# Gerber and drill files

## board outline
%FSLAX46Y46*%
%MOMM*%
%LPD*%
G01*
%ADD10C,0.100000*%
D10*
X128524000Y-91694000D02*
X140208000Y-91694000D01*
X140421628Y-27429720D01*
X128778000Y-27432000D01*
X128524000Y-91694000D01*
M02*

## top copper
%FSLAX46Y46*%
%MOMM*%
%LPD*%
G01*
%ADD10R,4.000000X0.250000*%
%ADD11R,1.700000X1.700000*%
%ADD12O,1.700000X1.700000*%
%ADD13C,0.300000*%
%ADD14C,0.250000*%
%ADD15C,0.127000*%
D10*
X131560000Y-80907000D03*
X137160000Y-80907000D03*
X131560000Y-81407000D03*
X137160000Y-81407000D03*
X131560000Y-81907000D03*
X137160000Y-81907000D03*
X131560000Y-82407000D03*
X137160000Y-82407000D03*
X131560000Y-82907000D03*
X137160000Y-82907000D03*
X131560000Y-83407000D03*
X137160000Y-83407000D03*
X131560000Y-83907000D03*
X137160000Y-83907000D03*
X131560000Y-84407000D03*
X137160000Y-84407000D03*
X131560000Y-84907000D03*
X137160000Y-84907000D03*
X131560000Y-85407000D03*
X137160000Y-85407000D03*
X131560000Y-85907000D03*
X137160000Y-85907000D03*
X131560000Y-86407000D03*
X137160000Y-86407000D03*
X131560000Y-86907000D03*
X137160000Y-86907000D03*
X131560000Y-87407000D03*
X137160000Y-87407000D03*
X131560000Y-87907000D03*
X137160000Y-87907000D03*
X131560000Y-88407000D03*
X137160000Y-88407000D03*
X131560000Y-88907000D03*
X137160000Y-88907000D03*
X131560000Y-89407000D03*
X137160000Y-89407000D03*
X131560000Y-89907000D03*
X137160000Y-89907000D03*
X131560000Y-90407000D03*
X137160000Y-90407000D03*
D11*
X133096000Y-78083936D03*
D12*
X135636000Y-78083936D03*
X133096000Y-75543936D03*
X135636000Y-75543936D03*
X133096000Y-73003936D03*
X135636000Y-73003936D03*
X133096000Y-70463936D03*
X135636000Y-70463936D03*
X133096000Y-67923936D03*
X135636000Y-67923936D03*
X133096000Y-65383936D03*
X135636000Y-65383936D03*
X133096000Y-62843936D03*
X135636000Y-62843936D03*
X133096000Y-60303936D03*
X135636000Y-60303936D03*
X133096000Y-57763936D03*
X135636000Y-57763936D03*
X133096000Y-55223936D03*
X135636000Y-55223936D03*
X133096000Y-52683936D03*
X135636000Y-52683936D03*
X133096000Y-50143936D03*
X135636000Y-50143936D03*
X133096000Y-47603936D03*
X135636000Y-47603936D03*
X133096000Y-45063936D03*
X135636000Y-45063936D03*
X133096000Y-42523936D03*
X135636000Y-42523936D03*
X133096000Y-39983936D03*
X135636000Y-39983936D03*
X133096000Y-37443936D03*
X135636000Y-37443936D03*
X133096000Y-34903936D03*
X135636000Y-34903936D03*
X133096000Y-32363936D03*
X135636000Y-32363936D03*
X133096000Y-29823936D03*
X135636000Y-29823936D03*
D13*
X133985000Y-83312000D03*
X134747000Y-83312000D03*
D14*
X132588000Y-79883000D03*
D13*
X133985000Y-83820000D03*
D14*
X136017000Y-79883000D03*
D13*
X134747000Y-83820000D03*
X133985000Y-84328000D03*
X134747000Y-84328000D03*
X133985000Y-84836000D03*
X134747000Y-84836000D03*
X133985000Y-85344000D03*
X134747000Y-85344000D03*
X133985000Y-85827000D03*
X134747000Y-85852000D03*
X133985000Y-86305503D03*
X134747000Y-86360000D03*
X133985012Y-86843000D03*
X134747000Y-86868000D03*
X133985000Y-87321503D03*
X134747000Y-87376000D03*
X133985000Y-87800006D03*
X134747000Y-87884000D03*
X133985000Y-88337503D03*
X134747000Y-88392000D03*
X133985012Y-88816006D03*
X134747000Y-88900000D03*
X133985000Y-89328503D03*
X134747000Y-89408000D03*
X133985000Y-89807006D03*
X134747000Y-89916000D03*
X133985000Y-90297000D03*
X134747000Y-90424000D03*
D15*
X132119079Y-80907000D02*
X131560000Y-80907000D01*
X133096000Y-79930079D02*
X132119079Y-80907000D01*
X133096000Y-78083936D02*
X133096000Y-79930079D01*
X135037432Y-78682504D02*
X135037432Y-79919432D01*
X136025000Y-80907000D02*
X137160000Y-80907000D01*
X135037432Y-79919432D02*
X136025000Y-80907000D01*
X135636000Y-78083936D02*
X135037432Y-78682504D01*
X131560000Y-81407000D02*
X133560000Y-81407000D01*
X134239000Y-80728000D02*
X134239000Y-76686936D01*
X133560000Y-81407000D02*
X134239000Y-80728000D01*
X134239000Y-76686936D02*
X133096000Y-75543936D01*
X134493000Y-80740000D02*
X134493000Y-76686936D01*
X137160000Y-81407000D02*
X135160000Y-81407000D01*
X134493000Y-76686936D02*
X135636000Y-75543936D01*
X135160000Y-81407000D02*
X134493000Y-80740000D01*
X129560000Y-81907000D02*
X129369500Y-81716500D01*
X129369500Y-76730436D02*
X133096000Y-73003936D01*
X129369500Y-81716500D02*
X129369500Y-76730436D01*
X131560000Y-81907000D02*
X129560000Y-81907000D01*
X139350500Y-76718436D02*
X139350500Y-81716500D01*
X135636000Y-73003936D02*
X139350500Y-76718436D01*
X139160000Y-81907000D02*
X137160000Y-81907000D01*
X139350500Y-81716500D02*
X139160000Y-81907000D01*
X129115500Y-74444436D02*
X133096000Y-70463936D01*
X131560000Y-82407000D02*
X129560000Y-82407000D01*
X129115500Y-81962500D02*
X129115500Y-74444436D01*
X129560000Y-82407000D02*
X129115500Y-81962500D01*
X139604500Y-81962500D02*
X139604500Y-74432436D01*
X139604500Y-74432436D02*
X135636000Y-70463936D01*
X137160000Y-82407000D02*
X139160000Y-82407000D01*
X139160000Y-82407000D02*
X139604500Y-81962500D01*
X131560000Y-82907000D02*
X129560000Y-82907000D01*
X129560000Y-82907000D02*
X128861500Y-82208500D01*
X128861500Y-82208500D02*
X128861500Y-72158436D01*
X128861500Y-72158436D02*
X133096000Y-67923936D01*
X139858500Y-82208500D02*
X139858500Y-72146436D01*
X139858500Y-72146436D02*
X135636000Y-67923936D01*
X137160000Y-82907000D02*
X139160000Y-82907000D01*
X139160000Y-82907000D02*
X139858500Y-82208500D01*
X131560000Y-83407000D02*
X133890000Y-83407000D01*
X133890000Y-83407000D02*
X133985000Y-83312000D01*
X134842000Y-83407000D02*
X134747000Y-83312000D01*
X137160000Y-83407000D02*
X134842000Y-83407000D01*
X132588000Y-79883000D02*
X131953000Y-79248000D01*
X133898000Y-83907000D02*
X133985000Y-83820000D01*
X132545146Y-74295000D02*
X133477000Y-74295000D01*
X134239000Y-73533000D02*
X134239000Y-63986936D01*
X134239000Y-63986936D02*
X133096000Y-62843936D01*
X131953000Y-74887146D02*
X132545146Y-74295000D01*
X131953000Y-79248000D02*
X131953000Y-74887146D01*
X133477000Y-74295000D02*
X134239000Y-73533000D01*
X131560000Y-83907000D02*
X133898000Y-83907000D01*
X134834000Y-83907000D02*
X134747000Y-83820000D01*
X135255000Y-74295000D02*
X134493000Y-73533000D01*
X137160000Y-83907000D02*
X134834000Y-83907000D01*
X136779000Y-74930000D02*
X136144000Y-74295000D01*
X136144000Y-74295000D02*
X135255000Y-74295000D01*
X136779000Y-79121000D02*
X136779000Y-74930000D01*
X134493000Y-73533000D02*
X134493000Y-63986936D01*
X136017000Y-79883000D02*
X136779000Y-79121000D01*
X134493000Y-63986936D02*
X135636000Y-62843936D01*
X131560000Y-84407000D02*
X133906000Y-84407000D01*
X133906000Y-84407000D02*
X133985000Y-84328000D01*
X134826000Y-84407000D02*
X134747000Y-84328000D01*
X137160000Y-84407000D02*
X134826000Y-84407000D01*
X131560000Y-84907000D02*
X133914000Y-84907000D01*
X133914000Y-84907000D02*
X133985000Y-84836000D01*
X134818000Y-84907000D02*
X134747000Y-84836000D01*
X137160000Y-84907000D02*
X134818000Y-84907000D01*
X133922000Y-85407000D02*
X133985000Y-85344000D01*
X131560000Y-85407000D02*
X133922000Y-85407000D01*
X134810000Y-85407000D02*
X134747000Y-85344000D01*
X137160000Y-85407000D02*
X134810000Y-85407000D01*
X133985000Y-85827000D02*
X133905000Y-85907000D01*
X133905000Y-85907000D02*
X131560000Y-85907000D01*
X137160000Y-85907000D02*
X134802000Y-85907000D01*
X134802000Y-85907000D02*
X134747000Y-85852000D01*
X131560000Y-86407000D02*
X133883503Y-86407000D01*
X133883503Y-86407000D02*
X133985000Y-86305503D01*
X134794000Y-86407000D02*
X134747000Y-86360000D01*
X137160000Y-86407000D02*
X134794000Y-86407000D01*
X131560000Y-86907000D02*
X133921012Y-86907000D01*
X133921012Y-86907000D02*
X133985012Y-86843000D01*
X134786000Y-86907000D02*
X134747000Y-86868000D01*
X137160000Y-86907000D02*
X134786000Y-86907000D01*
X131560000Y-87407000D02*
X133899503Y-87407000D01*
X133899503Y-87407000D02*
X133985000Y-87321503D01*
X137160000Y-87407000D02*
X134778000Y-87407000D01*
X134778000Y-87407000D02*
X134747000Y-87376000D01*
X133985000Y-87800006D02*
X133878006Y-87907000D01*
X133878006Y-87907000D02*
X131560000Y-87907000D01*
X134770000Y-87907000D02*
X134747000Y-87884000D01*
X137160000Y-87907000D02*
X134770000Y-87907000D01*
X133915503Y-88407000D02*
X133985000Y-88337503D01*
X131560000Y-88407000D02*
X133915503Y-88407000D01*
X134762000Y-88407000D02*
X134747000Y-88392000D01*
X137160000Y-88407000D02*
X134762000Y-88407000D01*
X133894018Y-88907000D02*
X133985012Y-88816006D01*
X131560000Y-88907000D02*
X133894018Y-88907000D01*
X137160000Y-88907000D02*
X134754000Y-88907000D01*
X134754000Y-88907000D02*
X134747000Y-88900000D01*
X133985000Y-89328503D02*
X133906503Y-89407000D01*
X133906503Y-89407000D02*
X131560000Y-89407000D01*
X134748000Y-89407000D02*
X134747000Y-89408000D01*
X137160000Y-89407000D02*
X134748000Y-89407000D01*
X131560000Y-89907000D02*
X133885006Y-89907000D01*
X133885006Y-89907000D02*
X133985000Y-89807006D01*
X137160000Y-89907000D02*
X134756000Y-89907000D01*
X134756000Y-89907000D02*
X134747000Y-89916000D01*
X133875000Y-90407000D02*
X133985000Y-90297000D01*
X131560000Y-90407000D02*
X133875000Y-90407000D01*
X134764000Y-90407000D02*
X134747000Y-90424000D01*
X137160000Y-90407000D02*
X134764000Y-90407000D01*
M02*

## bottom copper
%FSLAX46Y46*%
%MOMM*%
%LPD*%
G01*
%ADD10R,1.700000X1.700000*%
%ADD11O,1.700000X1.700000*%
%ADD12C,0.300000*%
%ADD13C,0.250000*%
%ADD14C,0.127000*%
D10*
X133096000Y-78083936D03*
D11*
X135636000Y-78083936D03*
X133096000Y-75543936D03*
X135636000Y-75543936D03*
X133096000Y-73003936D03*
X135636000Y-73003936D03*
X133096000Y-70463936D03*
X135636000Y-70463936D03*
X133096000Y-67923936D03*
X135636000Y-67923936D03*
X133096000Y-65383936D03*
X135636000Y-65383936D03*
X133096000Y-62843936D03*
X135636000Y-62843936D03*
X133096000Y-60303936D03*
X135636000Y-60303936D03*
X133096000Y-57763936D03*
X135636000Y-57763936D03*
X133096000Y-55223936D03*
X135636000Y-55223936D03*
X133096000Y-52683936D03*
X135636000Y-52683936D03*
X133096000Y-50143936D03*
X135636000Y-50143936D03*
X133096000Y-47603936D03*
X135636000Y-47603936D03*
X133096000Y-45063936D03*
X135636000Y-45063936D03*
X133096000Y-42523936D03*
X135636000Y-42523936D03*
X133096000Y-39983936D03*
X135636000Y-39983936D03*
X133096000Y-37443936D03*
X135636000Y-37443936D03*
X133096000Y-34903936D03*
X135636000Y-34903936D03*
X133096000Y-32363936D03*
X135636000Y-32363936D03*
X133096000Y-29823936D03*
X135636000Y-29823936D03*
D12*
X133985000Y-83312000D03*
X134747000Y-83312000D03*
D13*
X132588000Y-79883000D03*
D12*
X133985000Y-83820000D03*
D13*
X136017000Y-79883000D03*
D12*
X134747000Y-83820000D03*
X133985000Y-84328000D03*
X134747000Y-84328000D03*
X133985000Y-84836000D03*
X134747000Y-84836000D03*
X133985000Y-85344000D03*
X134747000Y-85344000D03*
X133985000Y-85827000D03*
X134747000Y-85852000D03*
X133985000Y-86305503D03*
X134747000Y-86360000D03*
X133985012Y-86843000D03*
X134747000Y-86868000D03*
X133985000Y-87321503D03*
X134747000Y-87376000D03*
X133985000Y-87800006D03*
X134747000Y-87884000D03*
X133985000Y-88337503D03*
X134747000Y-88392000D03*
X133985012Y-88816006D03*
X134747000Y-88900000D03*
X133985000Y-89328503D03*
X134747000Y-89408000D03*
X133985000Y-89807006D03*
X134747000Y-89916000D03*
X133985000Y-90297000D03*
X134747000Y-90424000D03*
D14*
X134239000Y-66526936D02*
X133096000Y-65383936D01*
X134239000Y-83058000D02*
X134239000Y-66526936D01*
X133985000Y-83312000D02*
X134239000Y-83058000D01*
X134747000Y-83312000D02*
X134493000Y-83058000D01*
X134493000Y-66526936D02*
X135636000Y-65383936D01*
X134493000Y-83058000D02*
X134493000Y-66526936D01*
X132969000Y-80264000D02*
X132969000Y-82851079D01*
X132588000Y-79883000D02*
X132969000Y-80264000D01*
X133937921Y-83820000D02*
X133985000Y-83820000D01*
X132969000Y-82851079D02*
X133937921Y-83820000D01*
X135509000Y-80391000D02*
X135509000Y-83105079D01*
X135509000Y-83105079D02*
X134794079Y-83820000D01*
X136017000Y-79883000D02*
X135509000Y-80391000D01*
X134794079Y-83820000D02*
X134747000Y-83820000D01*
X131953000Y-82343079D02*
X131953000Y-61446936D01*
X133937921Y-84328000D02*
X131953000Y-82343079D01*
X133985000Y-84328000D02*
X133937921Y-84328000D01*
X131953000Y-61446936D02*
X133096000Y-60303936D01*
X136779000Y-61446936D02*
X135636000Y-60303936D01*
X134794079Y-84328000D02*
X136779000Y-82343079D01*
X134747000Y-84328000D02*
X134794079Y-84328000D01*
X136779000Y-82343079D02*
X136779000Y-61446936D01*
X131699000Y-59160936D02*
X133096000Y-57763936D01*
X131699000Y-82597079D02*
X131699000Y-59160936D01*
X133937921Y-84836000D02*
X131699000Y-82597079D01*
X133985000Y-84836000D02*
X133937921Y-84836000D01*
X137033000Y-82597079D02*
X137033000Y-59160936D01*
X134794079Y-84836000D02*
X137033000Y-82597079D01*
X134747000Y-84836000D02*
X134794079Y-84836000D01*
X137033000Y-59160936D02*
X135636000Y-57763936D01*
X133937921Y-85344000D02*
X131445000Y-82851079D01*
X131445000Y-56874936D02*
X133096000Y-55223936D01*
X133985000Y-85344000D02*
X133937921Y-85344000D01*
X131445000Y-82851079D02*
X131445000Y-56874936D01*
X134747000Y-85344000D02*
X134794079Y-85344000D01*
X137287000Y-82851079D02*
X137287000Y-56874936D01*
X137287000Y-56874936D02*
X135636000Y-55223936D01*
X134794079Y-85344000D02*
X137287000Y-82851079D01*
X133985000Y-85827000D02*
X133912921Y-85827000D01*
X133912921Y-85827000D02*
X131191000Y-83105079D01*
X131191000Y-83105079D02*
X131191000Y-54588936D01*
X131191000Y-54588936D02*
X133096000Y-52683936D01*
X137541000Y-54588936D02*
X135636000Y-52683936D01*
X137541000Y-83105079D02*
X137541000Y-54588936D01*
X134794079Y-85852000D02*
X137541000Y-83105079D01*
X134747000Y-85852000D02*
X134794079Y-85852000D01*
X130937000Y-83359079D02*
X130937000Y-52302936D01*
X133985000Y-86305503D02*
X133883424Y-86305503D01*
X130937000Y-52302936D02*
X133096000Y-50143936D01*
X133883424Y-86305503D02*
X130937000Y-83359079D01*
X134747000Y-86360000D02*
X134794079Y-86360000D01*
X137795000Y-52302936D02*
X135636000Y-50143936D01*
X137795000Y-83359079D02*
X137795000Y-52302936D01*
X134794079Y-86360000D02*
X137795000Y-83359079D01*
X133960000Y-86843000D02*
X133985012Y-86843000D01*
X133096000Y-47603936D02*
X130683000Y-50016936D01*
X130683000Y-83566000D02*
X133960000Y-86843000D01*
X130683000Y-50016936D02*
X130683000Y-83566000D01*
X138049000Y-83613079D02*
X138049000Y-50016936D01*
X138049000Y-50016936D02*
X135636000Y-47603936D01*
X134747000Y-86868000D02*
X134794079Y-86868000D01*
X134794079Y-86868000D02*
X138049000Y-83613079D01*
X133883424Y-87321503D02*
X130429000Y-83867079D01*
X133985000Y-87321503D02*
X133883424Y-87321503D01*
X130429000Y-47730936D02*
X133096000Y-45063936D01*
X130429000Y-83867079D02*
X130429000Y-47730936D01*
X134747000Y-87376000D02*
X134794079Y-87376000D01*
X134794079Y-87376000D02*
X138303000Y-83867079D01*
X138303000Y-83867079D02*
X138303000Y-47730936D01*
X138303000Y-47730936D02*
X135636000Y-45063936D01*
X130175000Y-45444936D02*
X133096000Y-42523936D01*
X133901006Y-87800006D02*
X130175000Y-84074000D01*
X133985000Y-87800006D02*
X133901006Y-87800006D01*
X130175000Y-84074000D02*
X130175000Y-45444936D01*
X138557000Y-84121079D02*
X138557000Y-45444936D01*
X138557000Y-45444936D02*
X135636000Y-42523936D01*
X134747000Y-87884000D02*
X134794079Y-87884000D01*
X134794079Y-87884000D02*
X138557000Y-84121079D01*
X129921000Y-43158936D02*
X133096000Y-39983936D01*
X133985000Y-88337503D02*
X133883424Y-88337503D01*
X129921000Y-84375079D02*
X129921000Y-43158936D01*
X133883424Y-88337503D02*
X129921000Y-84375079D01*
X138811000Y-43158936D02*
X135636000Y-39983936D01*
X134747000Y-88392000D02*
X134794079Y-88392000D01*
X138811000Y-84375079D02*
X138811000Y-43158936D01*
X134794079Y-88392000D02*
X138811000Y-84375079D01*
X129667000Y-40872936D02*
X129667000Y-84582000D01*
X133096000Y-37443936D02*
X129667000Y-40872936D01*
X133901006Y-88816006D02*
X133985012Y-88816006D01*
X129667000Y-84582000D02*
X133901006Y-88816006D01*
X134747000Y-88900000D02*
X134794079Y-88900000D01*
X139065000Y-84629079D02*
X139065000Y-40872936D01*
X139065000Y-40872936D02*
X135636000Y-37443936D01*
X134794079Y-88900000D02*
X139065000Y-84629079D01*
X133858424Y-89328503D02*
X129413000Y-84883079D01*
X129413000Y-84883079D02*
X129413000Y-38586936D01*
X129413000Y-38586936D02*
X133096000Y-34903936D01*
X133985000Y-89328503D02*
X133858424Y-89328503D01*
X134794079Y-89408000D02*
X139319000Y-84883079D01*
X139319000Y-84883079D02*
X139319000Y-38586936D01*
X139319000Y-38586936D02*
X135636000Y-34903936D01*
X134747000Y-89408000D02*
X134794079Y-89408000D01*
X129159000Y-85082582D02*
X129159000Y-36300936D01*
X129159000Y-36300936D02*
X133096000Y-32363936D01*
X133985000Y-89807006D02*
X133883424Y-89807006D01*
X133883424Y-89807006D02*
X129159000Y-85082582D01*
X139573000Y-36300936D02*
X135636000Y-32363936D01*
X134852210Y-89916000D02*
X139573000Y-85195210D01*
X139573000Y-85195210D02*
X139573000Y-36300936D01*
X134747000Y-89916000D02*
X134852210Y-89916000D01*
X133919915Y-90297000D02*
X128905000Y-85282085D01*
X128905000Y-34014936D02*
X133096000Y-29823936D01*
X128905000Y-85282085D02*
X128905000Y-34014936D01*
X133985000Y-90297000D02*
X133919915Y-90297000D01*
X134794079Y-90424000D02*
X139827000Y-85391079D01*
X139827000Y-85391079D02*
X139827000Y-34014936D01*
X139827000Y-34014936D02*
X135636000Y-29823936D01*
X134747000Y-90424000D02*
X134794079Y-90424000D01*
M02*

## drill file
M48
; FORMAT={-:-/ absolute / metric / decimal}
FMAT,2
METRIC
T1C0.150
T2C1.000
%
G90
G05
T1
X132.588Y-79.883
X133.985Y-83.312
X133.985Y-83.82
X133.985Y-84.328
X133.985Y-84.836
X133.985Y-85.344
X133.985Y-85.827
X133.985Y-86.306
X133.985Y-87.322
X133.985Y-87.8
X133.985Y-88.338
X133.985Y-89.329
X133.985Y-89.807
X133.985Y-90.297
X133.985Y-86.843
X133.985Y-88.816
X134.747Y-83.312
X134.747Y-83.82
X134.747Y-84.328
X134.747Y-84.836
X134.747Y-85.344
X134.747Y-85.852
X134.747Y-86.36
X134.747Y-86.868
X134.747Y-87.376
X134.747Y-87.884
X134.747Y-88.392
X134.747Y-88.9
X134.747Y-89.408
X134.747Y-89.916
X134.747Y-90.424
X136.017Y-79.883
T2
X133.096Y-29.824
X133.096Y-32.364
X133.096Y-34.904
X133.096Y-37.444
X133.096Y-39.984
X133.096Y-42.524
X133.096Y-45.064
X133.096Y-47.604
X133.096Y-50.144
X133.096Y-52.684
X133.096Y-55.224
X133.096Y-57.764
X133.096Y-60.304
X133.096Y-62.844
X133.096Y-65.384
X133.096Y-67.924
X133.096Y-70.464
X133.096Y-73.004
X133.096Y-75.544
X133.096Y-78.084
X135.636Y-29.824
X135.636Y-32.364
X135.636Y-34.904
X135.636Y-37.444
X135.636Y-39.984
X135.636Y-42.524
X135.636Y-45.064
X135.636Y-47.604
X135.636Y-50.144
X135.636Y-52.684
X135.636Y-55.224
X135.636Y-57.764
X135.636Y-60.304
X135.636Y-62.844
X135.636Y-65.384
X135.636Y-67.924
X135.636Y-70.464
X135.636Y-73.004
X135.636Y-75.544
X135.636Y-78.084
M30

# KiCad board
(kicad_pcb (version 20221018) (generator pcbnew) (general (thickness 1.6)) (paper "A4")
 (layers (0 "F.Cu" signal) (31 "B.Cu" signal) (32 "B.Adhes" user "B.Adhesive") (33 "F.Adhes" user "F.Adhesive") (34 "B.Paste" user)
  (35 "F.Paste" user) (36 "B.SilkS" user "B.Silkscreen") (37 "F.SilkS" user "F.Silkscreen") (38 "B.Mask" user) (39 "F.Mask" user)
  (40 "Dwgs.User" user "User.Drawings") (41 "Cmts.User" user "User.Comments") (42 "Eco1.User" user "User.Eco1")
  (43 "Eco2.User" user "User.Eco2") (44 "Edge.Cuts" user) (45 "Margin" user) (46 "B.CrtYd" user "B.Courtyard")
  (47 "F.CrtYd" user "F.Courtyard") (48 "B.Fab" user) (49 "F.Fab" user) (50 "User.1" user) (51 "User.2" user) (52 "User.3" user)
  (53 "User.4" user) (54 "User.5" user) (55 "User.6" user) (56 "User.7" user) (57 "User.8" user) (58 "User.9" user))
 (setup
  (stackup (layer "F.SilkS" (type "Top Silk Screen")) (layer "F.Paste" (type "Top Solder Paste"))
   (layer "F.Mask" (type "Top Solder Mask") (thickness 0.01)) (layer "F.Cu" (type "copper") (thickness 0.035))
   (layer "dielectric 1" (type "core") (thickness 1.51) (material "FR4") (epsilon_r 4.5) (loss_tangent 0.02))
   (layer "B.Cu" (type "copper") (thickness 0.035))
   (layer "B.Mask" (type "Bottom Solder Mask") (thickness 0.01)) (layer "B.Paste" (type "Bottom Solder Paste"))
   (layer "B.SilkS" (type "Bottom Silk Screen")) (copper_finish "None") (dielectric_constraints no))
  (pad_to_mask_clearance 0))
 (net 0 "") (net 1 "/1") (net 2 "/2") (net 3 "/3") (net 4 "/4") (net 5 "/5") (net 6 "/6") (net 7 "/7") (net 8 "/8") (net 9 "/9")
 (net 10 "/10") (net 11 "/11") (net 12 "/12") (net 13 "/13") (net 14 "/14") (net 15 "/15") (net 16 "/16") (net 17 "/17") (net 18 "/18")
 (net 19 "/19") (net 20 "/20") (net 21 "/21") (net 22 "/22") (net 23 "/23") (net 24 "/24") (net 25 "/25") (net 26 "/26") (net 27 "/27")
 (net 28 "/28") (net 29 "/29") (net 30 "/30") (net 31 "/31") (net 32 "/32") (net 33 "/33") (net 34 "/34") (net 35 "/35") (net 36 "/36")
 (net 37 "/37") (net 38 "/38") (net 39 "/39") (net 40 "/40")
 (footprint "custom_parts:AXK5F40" (layer "F.Cu") (at 134.36 85.657)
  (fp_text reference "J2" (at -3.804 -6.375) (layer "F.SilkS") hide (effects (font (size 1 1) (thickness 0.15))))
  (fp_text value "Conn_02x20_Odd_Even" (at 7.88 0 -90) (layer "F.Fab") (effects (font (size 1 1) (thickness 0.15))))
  (pad "1" smd rect (at -2.8 -4.75 270) (size 0.25 4) (layers "F.Cu" "F.Paste" "F.Mask") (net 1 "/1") (thermal_bridge_angle 45))
  (pad "2" smd rect (at 2.8 -4.75 270) (size 0.25 4) (layers "F.Cu" "F.Paste" "F.Mask") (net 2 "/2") (thermal_bridge_angle 45))
  (pad "3" smd rect (at -2.8 -4.25 270) (size 0.25 4) (layers "F.Cu" "F.Paste" "F.Mask") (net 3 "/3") (thermal_bridge_angle 45))
  (pad "4" smd rect (at 2.8 -4.25 270) (size 0.25 4) (layers "F.Cu" "F.Paste" "F.Mask") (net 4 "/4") (thermal_bridge_angle 45))
  (pad "5" smd rect (at -2.8 -3.75 270) (size 0.25 4) (layers "F.Cu" "F.Paste" "F.Mask") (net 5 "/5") (thermal_bridge_angle 45))
  (pad "6" smd rect (at 2.8 -3.75 270) (size 0.25 4) (layers "F.Cu" "F.Paste" "F.Mask") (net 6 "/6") (thermal_bridge_angle 45))
  (pad "7" smd rect (at -2.8 -3.25 270) (size 0.25 4) (layers "F.Cu" "F.Paste" "F.Mask") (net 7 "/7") (thermal_bridge_angle 45))
  (pad "8" smd rect (at 2.8 -3.25 270) (size 0.25 4) (layers "F.Cu" "F.Paste" "F.Mask") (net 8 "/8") (thermal_bridge_angle 45))
  (pad "9" smd rect (at -2.8 -2.75 270) (size 0.25 4) (layers "F.Cu" "F.Paste" "F.Mask") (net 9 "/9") (thermal_bridge_angle 45))
  (pad "10" smd rect (at 2.8 -2.75 270) (size 0.25 4) (layers "F.Cu" "F.Paste" "F.Mask") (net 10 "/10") (thermal_bridge_angle 45))
  (pad "11" smd rect (at -2.8 -2.25 270) (size 0.25 4) (layers "F.Cu" "F.Paste" "F.Mask") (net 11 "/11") (thermal_bridge_angle 45))
  (pad "12" smd rect (at 2.8 -2.25 270) (size 0.25 4) (layers "F.Cu" "F.Paste" "F.Mask") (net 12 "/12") (thermal_bridge_angle 45))
  (pad "13" smd rect (at -2.8 -1.75 270) (size 0.25 4) (layers "F.Cu" "F.Paste" "F.Mask") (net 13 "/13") (thermal_bridge_angle 45))
  (pad "14" smd rect (at 2.8 -1.75 270) (size 0.25 4) (layers "F.Cu" "F.Paste" "F.Mask") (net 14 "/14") (thermal_bridge_angle 45))
  (pad "15" smd rect (at -2.8 -1.25 270) (size 0.25 4) (layers "F.Cu" "F.Paste" "F.Mask") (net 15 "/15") (thermal_bridge_angle 45))
  (pad "16" smd rect (at 2.8 -1.25 270) (size 0.25 4) (layers "F.Cu" "F.Paste" "F.Mask") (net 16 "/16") (thermal_bridge_angle 45))
  (pad "17" smd rect (at -2.8 -0.75 270) (size 0.25 4) (layers "F.Cu" "F.Paste" "F.Mask") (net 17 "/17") (thermal_bridge_angle 45))
  (pad "18" smd rect (at 2.8 -0.75 270) (size 0.25 4) (layers "F.Cu" "F.Paste" "F.Mask") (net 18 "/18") (thermal_bridge_angle 45))
  (pad "19" smd rect (at -2.8 -0.25 270) (size 0.25 4) (layers "F.Cu" "F.Paste" "F.Mask") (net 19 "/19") (thermal_bridge_angle 45))
  (pad "20" smd rect (at 2.8 -0.25 270) (size 0.25 4) (layers "F.Cu" "F.Paste" "F.Mask") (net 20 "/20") (thermal_bridge_angle 45))
  (pad "21" smd rect (at -2.8 0.25 270) (size 0.25 4) (layers "F.Cu" "F.Paste" "F.Mask") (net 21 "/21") (thermal_bridge_angle 45))
  (pad "22" smd rect (at 2.8 0.25 270) (size 0.25 4) (layers "F.Cu" "F.Paste" "F.Mask") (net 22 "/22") (thermal_bridge_angle 45))
  (pad "23" smd rect (at -2.8 0.75 270) (size 0.25 4) (layers "F.Cu" "F.Paste" "F.Mask") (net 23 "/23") (thermal_bridge_angle 45))
  (pad "24" smd rect (at 2.8 0.75 270) (size 0.25 4) (layers "F.Cu" "F.Paste" "F.Mask") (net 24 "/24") (thermal_bridge_angle 45))
  (pad "25" smd rect (at -2.8 1.25 270) (size 0.25 4) (layers "F.Cu" "F.Paste" "F.Mask") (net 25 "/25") (thermal_bridge_angle 45))
  (pad "26" smd rect (at 2.8 1.25 270) (size 0.25 4) (layers "F.Cu" "F.Paste" "F.Mask") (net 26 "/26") (thermal_bridge_angle 45))
  (pad "27" smd rect (at -2.8 1.75 270) (size 0.25 4) (layers "F.Cu" "F.Paste" "F.Mask") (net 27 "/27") (thermal_bridge_angle 45))
  (pad "28" smd rect (at 2.8 1.75 270) (size 0.25 4) (layers "F.Cu" "F.Paste" "F.Mask") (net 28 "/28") (thermal_bridge_angle 45))
  (pad "29" smd rect (at -2.8 2.25 270) (size 0.25 4) (layers "F.Cu" "F.Paste" "F.Mask") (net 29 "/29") (thermal_bridge_angle 45))
  (pad "30" smd rect (at 2.8 2.25 270) (size 0.25 4) (layers "F.Cu" "F.Paste" "F.Mask") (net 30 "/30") (thermal_bridge_angle 45))
  (pad "31" smd rect (at -2.8 2.75 270) (size 0.25 4) (layers "F.Cu" "F.Paste" "F.Mask") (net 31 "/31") (thermal_bridge_angle 45))
  (pad "32" smd rect (at 2.8 2.75 270) (size 0.25 4) (layers "F.Cu" "F.Paste" "F.Mask") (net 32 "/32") (thermal_bridge_angle 45))
  (pad "33" smd rect (at -2.8 3.25 270) (size 0.25 4) (layers "F.Cu" "F.Paste" "F.Mask") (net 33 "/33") (thermal_bridge_angle 45))
  (pad "34" smd rect (at 2.8 3.25 270) (size 0.25 4) (layers "F.Cu" "F.Paste" "F.Mask") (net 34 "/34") (thermal_bridge_angle 45))
  (pad "35" smd rect (at -2.8 3.75 270) (size 0.25 4) (layers "F.Cu" "F.Paste" "F.Mask") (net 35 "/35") (thermal_bridge_angle 45))
  (pad "36" smd rect (at 2.8 3.75 270) (size 0.25 4) (layers "F.Cu" "F.Paste" "F.Mask") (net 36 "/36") (thermal_bridge_angle 45))
  (pad "37" smd rect (at -2.8 4.25 270) (size 0.25 4) (layers "F.Cu" "F.Paste" "F.Mask") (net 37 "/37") (thermal_bridge_angle 45))
  (pad "38" smd rect (at 2.8 4.25 270) (size 0.25 4) (layers "F.Cu" "F.Paste" "F.Mask") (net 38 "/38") (thermal_bridge_angle 45))
  (pad "39" smd rect (at -2.8 4.75 270) (size 0.25 4) (layers "F.Cu" "F.Paste" "F.Mask") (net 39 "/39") (thermal_bridge_angle 45))
  (pad "40" smd rect (at 2.8 4.75 270) (size 0.25 4) (layers "F.Cu" "F.Paste" "F.Mask") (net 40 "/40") (thermal_bridge_angle 45)))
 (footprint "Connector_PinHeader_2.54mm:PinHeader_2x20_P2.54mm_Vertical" (layer "B.Cu") (at 133.096 78.083936)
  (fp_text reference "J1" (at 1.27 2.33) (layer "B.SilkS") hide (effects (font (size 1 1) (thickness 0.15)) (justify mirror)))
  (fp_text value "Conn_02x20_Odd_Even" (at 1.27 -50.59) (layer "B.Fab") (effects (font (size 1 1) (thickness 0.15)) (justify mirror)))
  (pad "1" thru_hole rect (at 0 0) (size 1.7 1.7) (drill 1) (layers "*.Cu" "*.Mask") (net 1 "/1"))
  (pad "2" thru_hole oval (at 2.54 0) (size 1.7 1.7) (drill 1) (layers "*.Cu" "*.Mask") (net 2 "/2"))
  (pad "3" thru_hole oval (at 0 -2.54) (size 1.7 1.7) (drill 1) (layers "*.Cu" "*.Mask") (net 3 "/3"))
  (pad "4" thru_hole oval (at 2.54 -2.54) (size 1.7 1.7) (drill 1) (layers "*.Cu" "*.Mask") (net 4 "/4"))
  (pad "5" thru_hole oval (at 0 -5.08) (size 1.7 1.7) (drill 1) (layers "*.Cu" "*.Mask") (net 5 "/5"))
  (pad "6" thru_hole oval (at 2.54 -5.08) (size 1.7 1.7) (drill 1) (layers "*.Cu" "*.Mask") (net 6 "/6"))
  (pad "7" thru_hole oval (at 0 -7.62) (size 1.7 1.7) (drill 1) (layers "*.Cu" "*.Mask") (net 7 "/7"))
  (pad "8" thru_hole oval (at 2.54 -7.62) (size 1.7 1.7) (drill 1) (layers "*.Cu" "*.Mask") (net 8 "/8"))
  (pad "9" thru_hole oval (at 0 -10.16) (size 1.7 1.7) (drill 1) (layers "*.Cu" "*.Mask") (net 9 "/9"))
  (pad "10" thru_hole oval (at 2.54 -10.16) (size 1.7 1.7) (drill 1) (layers "*.Cu" "*.Mask") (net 10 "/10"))
  (pad "11" thru_hole oval (at 0 -12.7) (size 1.7 1.7) (drill 1) (layers "*.Cu" "*.Mask") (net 11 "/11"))
  (pad "12" thru_hole oval (at 2.54 -12.7) (size 1.7 1.7) (drill 1) (layers "*.Cu" "*.Mask") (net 12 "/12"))
  (pad "13" thru_hole oval (at 0 -15.24) (size 1.7 1.7) (drill 1) (layers "*.Cu" "*.Mask") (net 13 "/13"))
  (pad "14" thru_hole oval (at 2.54 -15.24) (size 1.7 1.7) (drill 1) (layers "*.Cu" "*.Mask") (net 14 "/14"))
  (pad "15" thru_hole oval (at 0 -17.78) (size 1.7 1.7) (drill 1) (layers "*.Cu" "*.Mask") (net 15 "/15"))
  (pad "16" thru_hole oval (at 2.54 -17.78) (size 1.7 1.7) (drill 1) (layers "*.Cu" "*.Mask") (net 16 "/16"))
  (pad "17" thru_hole oval (at 0 -20.32) (size 1.7 1.7) (drill 1) (layers "*.Cu" "*.Mask") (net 17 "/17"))
  (pad "18" thru_hole oval (at 2.54 -20.32) (size 1.7 1.7) (drill 1) (layers "*.Cu" "*.Mask") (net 18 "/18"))
  (pad "19" thru_hole oval (at 0 -22.86) (size 1.7 1.7) (drill 1) (layers "*.Cu" "*.Mask") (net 19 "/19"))
  (pad "20" thru_hole oval (at 2.54 -22.86) (size 1.7 1.7) (drill 1) (layers "*.Cu" "*.Mask") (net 20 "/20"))
  (pad "21" thru_hole oval (at 0 -25.4) (size 1.7 1.7) (drill 1) (layers "*.Cu" "*.Mask") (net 21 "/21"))
  (pad "22" thru_hole oval (at 2.54 -25.4) (size 1.7 1.7) (drill 1) (layers "*.Cu" "*.Mask") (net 22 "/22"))
  (pad "23" thru_hole oval (at 0 -27.94) (size 1.7 1.7) (drill 1) (layers "*.Cu" "*.Mask") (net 23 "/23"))
  (pad "24" thru_hole oval (at 2.54 -27.94) (size 1.7 1.7) (drill 1) (layers "*.Cu" "*.Mask") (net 24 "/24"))
  (pad "25" thru_hole oval (at 0 -30.48) (size 1.7 1.7) (drill 1) (layers "*.Cu" "*.Mask") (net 25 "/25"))
  (pad "26" thru_hole oval (at 2.54 -30.48) (size 1.7 1.7) (drill 1) (layers "*.Cu" "*.Mask") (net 26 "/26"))
  (pad "27" thru_hole oval (at 0 -33.02) (size 1.7 1.7) (drill 1) (layers "*.Cu" "*.Mask") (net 27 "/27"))
  (pad "28" thru_hole oval (at 2.54 -33.02) (size 1.7 1.7) (drill 1) (layers "*.Cu" "*.Mask") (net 28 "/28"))
  (pad "29" thru_hole oval (at 0 -35.56) (size 1.7 1.7) (drill 1) (layers "*.Cu" "*.Mask") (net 29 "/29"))
  (pad "30" thru_hole oval (at 2.54 -35.56) (size 1.7 1.7) (drill 1) (layers "*.Cu" "*.Mask") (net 30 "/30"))
  (pad "31" thru_hole oval (at 0 -38.1) (size 1.7 1.7) (drill 1) (layers "*.Cu" "*.Mask") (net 31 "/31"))
  (pad "32" thru_hole oval (at 2.54 -38.1) (size 1.7 1.7) (drill 1) (layers "*.Cu" "*.Mask") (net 32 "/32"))
  (pad "33" thru_hole oval (at 0 -40.64) (size 1.7 1.7) (drill 1) (layers "*.Cu" "*.Mask") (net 33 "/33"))
  (pad "34" thru_hole oval (at 2.54 -40.64) (size 1.7 1.7) (drill 1) (layers "*.Cu" "*.Mask") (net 34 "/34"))
  (pad "35" thru_hole oval (at 0 -43.18) (size 1.7 1.7) (drill 1) (layers "*.Cu" "*.Mask") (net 35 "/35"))
  (pad "36" thru_hole oval (at 2.54 -43.18) (size 1.7 1.7) (drill 1) (layers "*.Cu" "*.Mask") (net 36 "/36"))
  (pad "37" thru_hole oval (at 0 -45.72) (size 1.7 1.7) (drill 1) (layers "*.Cu" "*.Mask") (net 37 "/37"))
  (pad "38" thru_hole oval (at 2.54 -45.72) (size 1.7 1.7) (drill 1) (layers "*.Cu" "*.Mask") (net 38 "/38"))
  (pad "39" thru_hole oval (at 0 -48.26) (size 1.7 1.7) (drill 1) (layers "*.Cu" "*.Mask") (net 39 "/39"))
  (pad "40" thru_hole oval (at 2.54 -48.26) (size 1.7 1.7) (drill 1) (layers "*.Cu" "*.Mask") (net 40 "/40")))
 (gr_poly
  (pts (xy 128.524 91.694) (xy 140.208 91.694) (xy 140.421628 27.42972) (xy 128.778 27.432)) (stroke (width 0.1) (type solid)) (fill none)
  (layer "Edge.Cuts"))
 (segment (start 132.119079 80.907) (end 131.56 80.907) (width 0.127) (layer "F.Cu") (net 1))
 (segment (start 133.096 79.930079) (end 132.119079 80.907) (width 0.127) (layer "F.Cu") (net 1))
 (segment (start 133.096 78.083936) (end 133.096 79.930079) (width 0.127) (layer "F.Cu") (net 1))
 (segment (start 135.037432 78.682504) (end 135.037432 79.919432) (width 0.127) (layer "F.Cu") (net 2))
 (segment (start 136.025 80.907) (end 137.16 80.907) (width 0.127) (layer "F.Cu") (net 2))
 (segment (start 135.037432 79.919432) (end 136.025 80.907) (width 0.127) (layer "F.Cu") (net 2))
 (segment (start 135.636 78.083936) (end 135.037432 78.682504) (width 0.127) (layer "F.Cu") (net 2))
 (segment (start 131.56 81.407) (end 133.56 81.407) (width 0.127) (layer "F.Cu") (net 3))
 (segment (start 134.239 80.728) (end 134.239 76.686936) (width 0.127) (layer "F.Cu") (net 3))
 (segment (start 133.56 81.407) (end 134.239 80.728) (width 0.127) (layer "F.Cu") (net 3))
 (segment (start 134.239 76.686936) (end 133.096 75.543936) (width 0.127) (layer "F.Cu") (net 3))
 (segment (start 134.493 80.74) (end 134.493 76.686936) (width 0.127) (layer "F.Cu") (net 4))
 (segment (start 137.16 81.407) (end 135.16 81.407) (width 0.127) (layer "F.Cu") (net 4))
 (segment (start 134.493 76.686936) (end 135.636 75.543936) (width 0.127) (layer "F.Cu") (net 4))
 (segment (start 135.16 81.407) (end 134.493 80.74) (width 0.127) (layer "F.Cu") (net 4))
 (segment (start 129.56 81.907) (end 129.3695 81.7165) (width 0.127) (layer "F.Cu") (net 5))
 (segment (start 129.3695 76.730436) (end 133.096 73.003936) (width 0.127) (layer "F.Cu") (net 5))
 (segment (start 129.3695 81.7165) (end 129.3695 76.730436) (width 0.127) (layer "F.Cu") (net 5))
 (segment (start 131.56 81.907) (end 129.56 81.907) (width 0.127) (layer "F.Cu") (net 5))
 (segment (start 139.3505 76.718436) (end 139.3505 81.7165) (width 0.127) (layer "F.Cu") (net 6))
 (segment (start 135.636 73.003936) (end 139.3505 76.718436) (width 0.127) (layer "F.Cu") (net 6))
 (segment (start 139.16 81.907) (end 137.16 81.907) (width 0.127) (layer "F.Cu") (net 6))
 (segment (start 139.3505 81.7165) (end 139.16 81.907) (width 0.127) (layer "F.Cu") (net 6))
 (segment (start 129.1155 74.444436) (end 133.096 70.463936) (width 0.127) (layer "F.Cu") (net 7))
 (segment (start 131.56 82.407) (end 129.56 82.407) (width 0.127) (layer "F.Cu") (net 7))
 (segment (start 129.1155 81.9625) (end 129.1155 74.444436) (width 0.127) (layer "F.Cu") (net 7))
 (segment (start 129.56 82.407) (end 129.1155 81.9625) (width 0.127) (layer "F.Cu") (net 7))
 (segment (start 139.6045 81.9625) (end 139.6045 74.432436) (width 0.127) (layer "F.Cu") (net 8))
 (segment (start 139.6045 74.432436) (end 135.636 70.463936) (width 0.127) (layer "F.Cu") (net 8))
 (segment (start 137.16 82.407) (end 139.16 82.407) (width 0.127) (layer "F.Cu") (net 8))
 (segment (start 139.16 82.407) (end 139.6045 81.9625) (width 0.127) (layer "F.Cu") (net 8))
 (segment (start 131.56 82.907) (end 129.56 82.907) (width 0.127) (layer "F.Cu") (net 9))
 (segment (start 129.56 82.907) (end 128.8615 82.2085) (width 0.127) (layer "F.Cu") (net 9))
 (segment (start 128.8615 82.2085) (end 128.8615 72.158436) (width 0.127) (layer "F.Cu") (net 9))
 (segment (start 128.8615 72.158436) (end 133.096 67.923936) (width 0.127) (layer "F.Cu") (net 9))
 (segment (start 139.8585 82.2085) (end 139.8585 72.146436) (width 0.127) (layer "F.Cu") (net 10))
 (segment (start 139.8585 72.146436) (end 135.636 67.923936) (width 0.127) (layer "F.Cu") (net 10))
 (segment (start 137.16 82.907) (end 139.16 82.907) (width 0.127) (layer "F.Cu") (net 10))
 (segment (start 139.16 82.907) (end 139.8585 82.2085) (width 0.127) (layer "F.Cu") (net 10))
 (segment (start 131.56 83.407) (end 133.89 83.407) (width 0.127) (layer "F.Cu") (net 11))
 (segment (start 133.89 83.407) (end 133.985 83.312) (width 0.127) (layer "F.Cu") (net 11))
 (via (at 133.985 83.312) (size 0.3) (drill 0.15) (layers "F.Cu" "B.Cu") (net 11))
 (segment (start 134.239 66.526936) (end 133.096 65.383936) (width 0.127) (layer "B.Cu") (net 11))
 (segment (start 134.239 83.058) (end 134.239 66.526936) (width 0.127) (layer "B.Cu") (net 11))
 (segment (start 133.985 83.312) (end 134.239 83.058) (width 0.127) (layer "B.Cu") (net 11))
 (segment (start 134.842 83.407) (end 134.747 83.312) (width 0.127) (layer "F.Cu") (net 12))
 (segment (start 137.16 83.407) (end 134.842 83.407) (width 0.127) (layer "F.Cu") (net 12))
 (via (at 134.747 83.312) (size 0.3) (drill 0.15) (layers "F.Cu" "B.Cu") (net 12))
 (segment (start 134.747 83.312) (end 134.493 83.058) (width 0.127) (layer "B.Cu") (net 12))
 (segment (start 134.493 66.526936) (end 135.636 65.383936) (width 0.127) (layer "B.Cu") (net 12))
 (segment (start 134.493 83.058) (end 134.493 66.526936) (width 0.127) (layer "B.Cu") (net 12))
 (segment (start 132.588 79.883) (end 131.953 79.248) (width 0.127) (layer "F.Cu") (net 13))
 (segment (start 133.898 83.907) (end 133.985 83.82) (width 0.127) (layer "F.Cu") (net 13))
 (segment (start 132.545146 74.295) (end 133.477 74.295) (width 0.127) (layer "F.Cu") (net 13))
 (segment (start 134.239 73.533) (end 134.239 63.986936) (width 0.127) (layer "F.Cu") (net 13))
 (segment (start 134.239 63.986936) (end 133.096 62.843936) (width 0.127) (layer "F.Cu") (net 13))
 (segment (start 131.953 74.887146) (end 132.545146 74.295) (width 0.127) (layer "F.Cu") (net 13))
 (segment (start 131.953 79.248) (end 131.953 74.887146) (width 0.127) (layer "F.Cu") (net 13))
 (segment (start 133.477 74.295) (end 134.239 73.533) (width 0.127) (layer "F.Cu") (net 13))
 (segment (start 131.56 83.907) (end 133.898 83.907) (width 0.127) (layer "F.Cu") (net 13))
 (via (at 132.588 79.883) (size 0.25) (drill 0.15) (layers "F.Cu" "B.Cu") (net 13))
 (via (at 133.985 83.82) (size 0.3) (drill 0.15) (layers "F.Cu" "B.Cu") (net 13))
 (segment (start 132.969 80.264) (end 132.969 82.851079) (width 0.127) (layer "B.Cu") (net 13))
 (segment (start 132.588 79.883) (end 132.969 80.264) (width 0.127) (layer "B.Cu") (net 13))
 (segment (start 133.937921 83.82) (end 133.985 83.82) (width 0.127) (layer "B.Cu") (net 13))
 (segment (start 132.969 82.851079) (end 133.937921 83.82) (width 0.127) (layer "B.Cu") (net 13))
 (segment (start 134.834 83.907) (end 134.747 83.82) (width 0.127) (layer "F.Cu") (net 14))
 (segment (start 135.255 74.295) (end 134.493 73.533) (width 0.127) (layer "F.Cu") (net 14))
 (segment (start 137.16 83.907) (end 134.834 83.907) (width 0.127) (layer "F.Cu") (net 14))
 (segment (start 136.779 74.93) (end 136.144 74.295) (width 0.127) (layer "F.Cu") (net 14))
 (segment (start 136.144 74.295) (end 135.255 74.295) (width 0.127) (layer "F.Cu") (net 14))
 (segment (start 136.779 79.121) (end 136.779 74.93) (width 0.127) (layer "F.Cu") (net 14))
 (segment (start 134.493 73.533) (end 134.493 63.986936) (width 0.127) (layer "F.Cu") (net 14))
 (segment (start 136.017 79.883) (end 136.779 79.121) (width 0.127) (layer "F.Cu") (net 14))
 (segment (start 134.493 63.986936) (end 135.636 62.843936) (width 0.127) (layer "F.Cu") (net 14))
 (via (at 136.017 79.883) (size 0.25) (drill 0.15) (layers "F.Cu" "B.Cu") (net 14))
 (via (at 134.747 83.82) (size 0.3) (drill 0.15) (layers "F.Cu" "B.Cu") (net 14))
 (segment (start 135.509 80.391) (end 135.509 83.105079) (width 0.127) (layer "B.Cu") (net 14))
 (segment (start 135.509 83.105079) (end 134.794079 83.82) (width 0.127) (layer "B.Cu") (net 14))
 (segment (start 136.017 79.883) (end 135.509 80.391) (width 0.127) (layer "B.Cu") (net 14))
 (segment (start 134.794079 83.82) (end 134.747 83.82) (width 0.127) (layer "B.Cu") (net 14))
 (segment (start 131.56 84.407) (end 133.906 84.407) (width 0.127) (layer "F.Cu") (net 15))
 (segment (start 133.906 84.407) (end 133.985 84.328) (width 0.127) (layer "F.Cu") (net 15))
 (via (at 133.985 84.328) (size 0.3) (drill 0.15) (layers "F.Cu" "B.Cu") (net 15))
 (segment (start 131.953 82.343079) (end 131.953 61.446936) (width 0.127) (layer "B.Cu") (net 15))
 (segment (start 133.937921 84.328) (end 131.953 82.343079) (width 0.127) (layer "B.Cu") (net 15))
 (segment (start 133.985 84.328) (end 133.937921 84.328) (width 0.127) (layer "B.Cu") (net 15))
 (segment (start 131.953 61.446936) (end 133.096 60.303936) (width 0.127) (layer "B.Cu") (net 15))
 (segment (start 134.826 84.407) (end 134.747 84.328) (width 0.127) (layer "F.Cu") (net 16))
 (segment (start 137.16 84.407) (end 134.826 84.407) (width 0.127) (layer "F.Cu") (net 16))
 (via (at 134.747 84.328) (size 0.3) (drill 0.15) (layers "F.Cu" "B.Cu") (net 16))
 (segment (start 136.779 61.446936) (end 135.636 60.303936) (width 0.127) (layer "B.Cu") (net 16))
 (segment (start 134.794079 84.328) (end 136.779 82.343079) (width 0.127) (layer "B.Cu") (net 16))
 (segment (start 134.747 84.328) (end 134.794079 84.328) (width 0.127) (layer "B.Cu") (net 16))
 (segment (start 136.779 82.343079) (end 136.779 61.446936) (width 0.127) (layer "B.Cu") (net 16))
 (segment (start 131.56 84.907) (end 133.914 84.907) (width 0.127) (layer "F.Cu") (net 17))
 (segment (start 133.914 84.907) (end 133.985 84.836) (width 0.127) (layer "F.Cu") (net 17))
 (via (at 133.985 84.836) (size 0.3) (drill 0.15) (layers "F.Cu" "B.Cu") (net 17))
 (segment (start 131.699 59.160936) (end 133.096 57.763936) (width 0.127) (layer "B.Cu") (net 17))
 (segment (start 131.699 82.597079) (end 131.699 59.160936) (width 0.127) (layer "B.Cu") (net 17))
 (segment (start 133.937921 84.836) (end 131.699 82.597079) (width 0.127) (layer "B.Cu") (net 17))
 (segment (start 133.985 84.836) (end 133.937921 84.836) (width 0.127) (layer "B.Cu") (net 17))
 (segment (start 134.818 84.907) (end 134.747 84.836) (width 0.127) (layer "F.Cu") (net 18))
 (segment (start 137.16 84.907) (end 134.818 84.907) (width 0.127) (layer "F.Cu") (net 18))
 (via (at 134.747 84.836) (size 0.3) (drill 0.15) (layers "F.Cu" "B.Cu") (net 18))
 (segment (start 137.033 82.597079) (end 137.033 59.160936) (width 0.127) (layer "B.Cu") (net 18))
 (segment (start 134.794079 84.836) (end 137.033 82.597079) (width 0.127) (layer "B.Cu") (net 18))
 (segment (start 134.747 84.836) (end 134.794079 84.836) (width 0.127) (layer "B.Cu") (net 18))
 (segment (start 137.033 59.160936) (end 135.636 57.763936) (width 0.127) (layer "B.Cu") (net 18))
 (segment (start 133.922 85.407) (end 133.985 85.344) (width 0.127) (layer "F.Cu") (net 19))
 (segment (start 131.56 85.407) (end 133.922 85.407) (width 0.127) (layer "F.Cu") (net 19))
 (via (at 133.985 85.344) (size 0.3) (drill 0.15) (layers "F.Cu" "B.Cu") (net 19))
 (segment (start 133.937921 85.344) (end 131.445 82.851079) (width 0.127) (layer "B.Cu") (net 19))
 (segment (start 131.445 56.874936) (end 133.096 55.223936) (width 0.127) (layer "B.Cu") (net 19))
 (segment (start 133.985 85.344) (end 133.937921 85.344) (width 0.127) (layer "B.Cu") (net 19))
 (segment (start 131.445 82.851079) (end 131.445 56.874936) (width 0.127) (layer "B.Cu") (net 19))
 (segment (start 134.81 85.407) (end 134.747 85.344) (width 0.127) (layer "F.Cu") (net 20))
 (segment (start 137.16 85.407) (end 134.81 85.407) (width 0.127) (layer "F.Cu") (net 20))
 (via (at 134.747 85.344) (size 0.3) (drill 0.15) (layers "F.Cu" "B.Cu") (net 20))
 (segment (start 134.747 85.344) (end 134.794079 85.344) (width 0.127) (layer "B.Cu") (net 20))
 (segment (start 137.287 82.851079) (end 137.287 56.874936) (width 0.127) (layer "B.Cu") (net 20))
 (segment (start 137.287 56.874936) (end 135.636 55.223936) (width 0.127) (layer "B.Cu") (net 20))
 (segment (start 134.794079 85.344) (end 137.287 82.851079) (width 0.127) (layer "B.Cu") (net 20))
 (segment (start 133.985 85.827) (end 133.905 85.907) (width 0.127) (layer "F.Cu") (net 21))
 (segment (start 133.905 85.907) (end 131.56 85.907) (width 0.127) (layer "F.Cu") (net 21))
 (via (at 133.985 85.827) (size 0.3) (drill 0.15) (layers "F.Cu" "B.Cu") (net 21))
 (segment (start 133.985 85.827) (end 133.912921 85.827) (width 0.127) (layer "B.Cu") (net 21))
 (segment (start 133.912921 85.827) (end 131.191 83.105079) (width 0.127) (layer "B.Cu") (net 21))
 (segment (start 131.191 83.105079) (end 131.191 54.588936) (width 0.127) (layer "B.Cu") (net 21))
 (segment (start 131.191 54.588936) (end 133.096 52.683936) (width 0.127) (layer "B.Cu") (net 21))
 (segment (start 137.16 85.907) (end 134.802 85.907) (width 0.127) (layer "F.Cu") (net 22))
 (segment (start 134.802 85.907) (end 134.747 85.852) (width 0.127) (layer "F.Cu") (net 22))
 (via (at 134.747 85.852) (size 0.3) (drill 0.15) (layers "F.Cu" "B.Cu") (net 22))
 (segment (start 137.541 54.588936) (end 135.636 52.683936) (width 0.127) (layer "B.Cu") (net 22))
 (segment (start 137.541 83.105079) (end 137.541 54.588936) (width 0.127) (layer "B.Cu") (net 22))
 (segment (start 134.794079 85.852) (end 137.541 83.105079) (width 0.127) (layer "B.Cu") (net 22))
 (segment (start 134.747 85.852) (end 134.794079 85.852) (width 0.127) (layer "B.Cu") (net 22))
 (segment (start 131.56 86.407) (end 133.883503 86.407) (width 0.127) (layer "F.Cu") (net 23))
 (segment (start 133.883503 86.407) (end 133.985 86.305503) (width 0.127) (layer "F.Cu") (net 23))
 (via (at 133.985 86.305503) (size 0.3) (drill 0.15) (layers "F.Cu" "B.Cu") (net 23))
 (segment (start 130.937 83.359079) (end 130.937 52.302936) (width 0.127) (layer "B.Cu") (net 23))
 (segment (start 133.985 86.305503) (end 133.883424 86.305503) (width 0.127) (layer "B.Cu") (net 23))
 (segment (start 130.937 52.302936) (end 133.096 50.143936) (width 0.127) (layer "B.Cu") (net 23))
 (segment (start 133.883424 86.305503) (end 130.937 83.359079) (width 0.127) (layer "B.Cu") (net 23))
 (segment (start 134.794 86.407) (end 134.747 86.36) (width 0.127) (layer "F.Cu") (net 24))
 (segment (start 137.16 86.407) (end 134.794 86.407) (width 0.127) (layer "F.Cu") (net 24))
 (via (at 134.747 86.36) (size 0.3) (drill 0.15) (layers "F.Cu" "B.Cu") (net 24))
 (segment (start 134.747 86.36) (end 134.794079 86.36) (width 0.127) (layer "B.Cu") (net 24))
 (segment (start 137.795 52.302936) (end 135.636 50.143936) (width 0.127) (layer "B.Cu") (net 24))
 (segment (start 137.795 83.359079) (end 137.795 52.302936) (width 0.127) (layer "B.Cu") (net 24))
 (segment (start 134.794079 86.36) (end 137.795 83.359079) (width 0.127) (layer "B.Cu") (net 24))
 (segment (start 131.56 86.907) (end 133.921012 86.907) (width 0.127) (layer "F.Cu") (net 25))
 (segment (start 133.921012 86.907) (end 133.985012 86.843) (width 0.127) (layer "F.Cu") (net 25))
 (via (at 133.985012 86.843) (size 0.3) (drill 0.15) (layers "F.Cu" "B.Cu") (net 25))
 (segment (start 133.96 86.843) (end 133.985012 86.843) (width 0.127) (layer "B.Cu") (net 25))
 (segment (start 133.096 47.603936) (end 130.683 50.016936) (width 0.127) (layer "B.Cu") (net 25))
 (segment (start 130.683 83.566) (end 133.96 86.843) (width 0.127) (layer "B.Cu") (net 25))
 (segment (start 130.683 50.016936) (end 130.683 83.566) (width 0.127) (layer "B.Cu") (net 25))
 (segment (start 134.786 86.907) (end 134.747 86.868) (width 0.127) (layer "F.Cu") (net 26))
 (segment (start 137.16 86.907) (end 134.786 86.907) (width 0.127) (layer "F.Cu") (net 26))
 (via (at 134.747 86.868) (size 0.3) (drill 0.15) (layers "F.Cu" "B.Cu") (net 26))
 (segment (start 138.049 83.613079) (end 138.049 50.016936) (width 0.127) (layer "B.Cu") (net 26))
 (segment (start 138.049 50.016936) (end 135.636 47.603936) (width 0.127) (layer "B.Cu") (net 26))
 (segment (start 134.747 86.868) (end 134.794079 86.868) (width 0.127) (layer "B.Cu") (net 26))
 (segment (start 134.794079 86.868) (end 138.049 83.613079) (width 0.127) (layer "B.Cu") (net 26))
 (segment (start 131.56 87.407) (end 133.899503 87.407) (width 0.127) (layer "F.Cu") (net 27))
 (segment (start 133.899503 87.407) (end 133.985 87.321503) (width 0.127) (layer "F.Cu") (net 27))
 (via (at 133.985 87.321503) (size 0.3) (drill 0.15) (layers "F.Cu" "B.Cu") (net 27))
 (segment (start 133.883424 87.321503) (end 130.429 83.867079) (width 0.127) (layer "B.Cu") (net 27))
 (segment (start 133.985 87.321503) (end 133.883424 87.321503) (width 0.127) (layer "B.Cu") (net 27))
 (segment (start 130.429 47.730936) (end 133.096 45.063936) (width 0.127) (layer "B.Cu") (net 27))
 (segment (start 130.429 83.867079) (end 130.429 47.730936) (width 0.127) (layer "B.Cu") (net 27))
 (segment (start 137.16 87.407) (end 134.778 87.407) (width 0.127) (layer "F.Cu") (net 28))
 (segment (start 134.778 87.407) (end 134.747 87.376) (width 0.127) (layer "F.Cu") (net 28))
 (via (at 134.747 87.376) (size 0.3) (drill 0.15) (layers "F.Cu" "B.Cu") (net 28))
 (segment (start 134.747 87.376) (end 134.794079 87.376) (width 0.127) (layer "B.Cu") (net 28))
 (segment (start 134.794079 87.376) (end 138.303 83.867079) (width 0.127) (layer "B.Cu") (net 28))
 (segment (start 138.303 83.867079) (end 138.303 47.730936) (width 0.127) (layer "B.Cu") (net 28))
 (segment (start 138.303 47.730936) (end 135.636 45.063936) (width 0.127) (layer "B.Cu") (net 28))
 (segment (start 133.985 87.800006) (end 133.878006 87.907) (width 0.127) (layer "F.Cu") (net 29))
 (segment (start 133.878006 87.907) (end 131.56 87.907) (width 0.127) (layer "F.Cu") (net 29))
 (via (at 133.985 87.800006) (size 0.3) (drill 0.15) (layers "F.Cu" "B.Cu") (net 29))
 (segment (start 130.175 45.444936) (end 133.096 42.523936) (width 0.127) (layer "B.Cu") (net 29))
 (segment (start 133.901006 87.800006) (end 130.175 84.074) (width 0.127) (layer "B.Cu") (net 29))
 (segment (start 133.985 87.800006) (end 133.901006 87.800006) (width 0.127) (layer "B.Cu") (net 29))
 (segment (start 130.175 84.074) (end 130.175 45.444936) (width 0.127) (layer "B.Cu") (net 29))
 (segment (start 134.77 87.907) (end 134.747 87.884) (width 0.127) (layer "F.Cu") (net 30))
 (segment (start 137.16 87.907) (end 134.77 87.907) (width 0.127) (layer "F.Cu") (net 30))
 (via (at 134.747 87.884) (size 0.3) (drill 0.15) (layers "F.Cu" "B.Cu") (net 30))
 (segment (start 138.557 84.121079) (end 138.557 45.444936) (width 0.127) (layer "B.Cu") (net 30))
 (segment (start 138.557 45.444936) (end 135.636 42.523936) (width 0.127) (layer "B.Cu") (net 30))
 (segment (start 134.747 87.884) (end 134.794079 87.884) (width 0.127) (layer "B.Cu") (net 30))
 (segment (start 134.794079 87.884) (end 138.557 84.121079) (width 0.127) (layer "B.Cu") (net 30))
 (segment (start 133.915503 88.407) (end 133.985 88.337503) (width 0.127) (layer "F.Cu") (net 31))
 (segment (start 131.56 88.407) (end 133.915503 88.407) (width 0.127) (layer "F.Cu") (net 31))
 (via (at 133.985 88.337503) (size 0.3) (drill 0.15) (layers "F.Cu" "B.Cu") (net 31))
 (segment (start 129.921 43.158936) (end 133.096 39.983936) (width 0.127) (layer "B.Cu") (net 31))
 (segment (start 133.985 88.337503) (end 133.883424 88.337503) (width 0.127) (layer "B.Cu") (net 31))
 (segment (start 129.921 84.375079) (end 129.921 43.158936) (width 0.127) (layer "B.Cu") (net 31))
 (segment (start 133.883424 88.337503) (end 129.921 84.375079) (width 0.127) (layer "B.Cu") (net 31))
 (segment (start 134.762 88.407) (end 134.747 88.392) (width 0.127) (layer "F.Cu") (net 32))
 (segment (start 137.16 88.407) (end 134.762 88.407) (width 0.127) (layer "F.Cu") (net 32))
 (via (at 134.747 88.392) (size 0.3) (drill 0.15) (layers "F.Cu" "B.Cu") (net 32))
 (segment (start 138.811 43.158936) (end 135.636 39.983936) (width 0.127) (layer "B.Cu") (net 32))
 (segment (start 134.747 88.392) (end 134.794079 88.392) (width 0.127) (layer "B.Cu") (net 32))
 (segment (start 138.811 84.375079) (end 138.811 43.158936) (width 0.127) (layer "B.Cu") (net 32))
 (segment (start 134.794079 88.392) (end 138.811 84.375079) (width 0.127) (layer "B.Cu") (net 32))
 (segment (start 133.894018 88.907) (end 133.985012 88.816006) (width 0.127) (layer "F.Cu") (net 33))
 (segment (start 131.56 88.907) (end 133.894018 88.907) (width 0.127) (layer "F.Cu") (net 33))
 (via (at 133.985012 88.816006) (size 0.3) (drill 0.15) (layers "F.Cu" "B.Cu") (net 33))
 (segment (start 129.667 40.872936) (end 129.667 84.582) (width 0.127) (layer "B.Cu") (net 33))
 (segment (start 133.096 37.443936) (end 129.667 40.872936) (width 0.127) (layer "B.Cu") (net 33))
 (segment (start 133.901006 88.816006) (end 133.985012 88.816006) (width 0.127) (layer "B.Cu") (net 33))
 (segment (start 129.667 84.582) (end 133.901006 88.816006) (width 0.127) (layer "B.Cu") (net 33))
 (segment (start 137.16 88.907) (end 134.754 88.907) (width 0.127) (layer "F.Cu") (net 34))
 (segment (start 134.754 88.907) (end 134.747 88.9) (width 0.127) (layer "F.Cu") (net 34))
 (via (at 134.747 88.9) (size 0.3) (drill 0.15) (layers "F.Cu" "B.Cu") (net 34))
 (segment (start 134.747 88.9) (end 134.794079 88.9) (width 0.127) (layer "B.Cu") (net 34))
 (segment (start 139.065 84.629079) (end 139.065 40.872936) (width 0.127) (layer "B.Cu") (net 34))
 (segment (start 139.065 40.872936) (end 135.636 37.443936) (width 0.127) (layer "B.Cu") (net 34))
 (segment (start 134.794079 88.9) (end 139.065 84.629079) (width 0.127) (layer "B.Cu") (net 34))
 (segment (start 133.985 89.328503) (end 133.906503 89.407) (width 0.127) (layer "F.Cu") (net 35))
 (segment (start 133.906503 89.407) (end 131.56 89.407) (width 0.127) (layer "F.Cu") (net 35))
 (via (at 133.985 89.328503) (size 0.3) (drill 0.15) (layers "F.Cu" "B.Cu") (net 35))
 (segment (start 133.858424 89.328503) (end 129.413 84.883079) (width 0.127) (layer "B.Cu") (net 35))
 (segment (start 129.413 84.883079) (end 129.413 38.586936) (width 0.127) (layer "B.Cu") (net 35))
 (segment (start 129.413 38.586936) (end 133.096 34.903936) (width 0.127) (layer "B.Cu") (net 35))
 (segment (start 133.985 89.328503) (end 133.858424 89.328503) (width 0.127) (layer "B.Cu") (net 35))
 (segment (start 134.748 89.407) (end 134.747 89.408) (width 0.127) (layer "F.Cu") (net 36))
 (segment (start 137.16 89.407) (end 134.748 89.407) (width 0.127) (layer "F.Cu") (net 36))
 (via (at 134.747 89.408) (size 0.3) (drill 0.15) (layers "F.Cu" "B.Cu") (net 36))
 (segment (start 134.794079 89.408) (end 139.319 84.883079) (width 0.127) (layer "B.Cu") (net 36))
 (segment (start 139.319 84.883079) (end 139.319 38.586936) (width 0.127) (layer "B.Cu") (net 36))
 (segment (start 139.319 38.586936) (end 135.636 34.903936) (width 0.127) (layer "B.Cu") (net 36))
 (segment (start 134.747 89.408) (end 134.794079 89.408) (width 0.127) (layer "B.Cu") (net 36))
 (segment (start 131.56 89.907) (end 133.885006 89.907) (width 0.127) (layer "F.Cu") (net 37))
 (segment (start 133.885006 89.907) (end 133.985 89.807006) (width 0.127) (layer "F.Cu") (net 37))
 (via (at 133.985 89.807006) (size 0.3) (drill 0.15) (layers "F.Cu" "B.Cu") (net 37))
 (segment (start 129.159 85.082582) (end 129.159 36.300936) (width 0.127) (layer "B.Cu") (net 37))
 (segment (start 129.159 36.300936) (end 133.096 32.363936) (width 0.127) (layer "B.Cu") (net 37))
 (segment (start 133.985 89.807006) (end 133.883424 89.807006) (width 0.127) (layer "B.Cu") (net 37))
 (segment (start 133.883424 89.807006) (end 129.159 85.082582) (width 0.127) (layer "B.Cu") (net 37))
 (segment (start 137.16 89.907) (end 134.756 89.907) (width 0.127) (layer "F.Cu") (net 38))
 (segment (start 134.756 89.907) (end 134.747 89.916) (width 0.127) (layer "F.Cu") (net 38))
 (via (at 134.747 89.916) (size 0.3) (drill 0.15) (layers "F.Cu" "B.Cu") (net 38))
 (segment (start 139.573 36.300936) (end 135.636 32.363936) (width 0.127) (layer "B.Cu") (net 38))
 (segment (start 134.85221 89.916) (end 139.573 85.19521) (width 0.127) (layer "B.Cu") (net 38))
 (segment (start 139.573 85.19521) (end 139.573 36.300936) (width 0.127) (layer "B.Cu") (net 38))
 (segment (start 134.747 89.916) (end 134.85221 89.916) (width 0.127) (layer "B.Cu") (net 38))
 (segment (start 133.875 90.407) (end 133.985 90.297) (width 0.127) (layer "F.Cu") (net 39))
 (segment (start 131.56 90.407) (end 133.875 90.407) (width 0.127) (layer "F.Cu") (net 39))
 (via (at 133.985 90.297) (size 0.3) (drill 0.15) (layers "F.Cu" "B.Cu") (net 39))
 (segment (start 133.919915 90.297) (end 128.905 85.282085) (width 0.127) (layer "B.Cu") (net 39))
 (segment (start 128.905 34.014936) (end 133.096 29.823936) (width 0.127) (layer "B.Cu") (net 39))
 (segment (start 128.905 85.282085) (end 128.905 34.014936) (width 0.127) (layer "B.Cu") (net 39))
 (segment (start 133.985 90.297) (end 133.919915 90.297) (width 0.127) (layer "B.Cu") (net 39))
 (segment (start 134.764 90.407) (end 134.747 90.424) (width 0.127) (layer "F.Cu") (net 40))
 (segment (start 137.16 90.407) (end 134.764 90.407) (width 0.127) (layer "F.Cu") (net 40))
 (via (at 134.747 90.424) (size 0.3) (drill 0.15) (layers "F.Cu" "B.Cu") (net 40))
 (segment (start 134.794079 90.424) (end 139.827 85.391079) (width 0.127) (layer "B.Cu") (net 40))
 (segment (start 139.827 85.391079) (end 139.827 34.014936) (width 0.127) (layer "B.Cu") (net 40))
 (segment (start 139.827 34.014936) (end 135.636 29.823936) (width 0.127) (layer "B.Cu") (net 40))
 (segment (start 134.747 90.424) (end 134.794079 90.424) (width 0.127) (layer "B.Cu") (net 40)))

